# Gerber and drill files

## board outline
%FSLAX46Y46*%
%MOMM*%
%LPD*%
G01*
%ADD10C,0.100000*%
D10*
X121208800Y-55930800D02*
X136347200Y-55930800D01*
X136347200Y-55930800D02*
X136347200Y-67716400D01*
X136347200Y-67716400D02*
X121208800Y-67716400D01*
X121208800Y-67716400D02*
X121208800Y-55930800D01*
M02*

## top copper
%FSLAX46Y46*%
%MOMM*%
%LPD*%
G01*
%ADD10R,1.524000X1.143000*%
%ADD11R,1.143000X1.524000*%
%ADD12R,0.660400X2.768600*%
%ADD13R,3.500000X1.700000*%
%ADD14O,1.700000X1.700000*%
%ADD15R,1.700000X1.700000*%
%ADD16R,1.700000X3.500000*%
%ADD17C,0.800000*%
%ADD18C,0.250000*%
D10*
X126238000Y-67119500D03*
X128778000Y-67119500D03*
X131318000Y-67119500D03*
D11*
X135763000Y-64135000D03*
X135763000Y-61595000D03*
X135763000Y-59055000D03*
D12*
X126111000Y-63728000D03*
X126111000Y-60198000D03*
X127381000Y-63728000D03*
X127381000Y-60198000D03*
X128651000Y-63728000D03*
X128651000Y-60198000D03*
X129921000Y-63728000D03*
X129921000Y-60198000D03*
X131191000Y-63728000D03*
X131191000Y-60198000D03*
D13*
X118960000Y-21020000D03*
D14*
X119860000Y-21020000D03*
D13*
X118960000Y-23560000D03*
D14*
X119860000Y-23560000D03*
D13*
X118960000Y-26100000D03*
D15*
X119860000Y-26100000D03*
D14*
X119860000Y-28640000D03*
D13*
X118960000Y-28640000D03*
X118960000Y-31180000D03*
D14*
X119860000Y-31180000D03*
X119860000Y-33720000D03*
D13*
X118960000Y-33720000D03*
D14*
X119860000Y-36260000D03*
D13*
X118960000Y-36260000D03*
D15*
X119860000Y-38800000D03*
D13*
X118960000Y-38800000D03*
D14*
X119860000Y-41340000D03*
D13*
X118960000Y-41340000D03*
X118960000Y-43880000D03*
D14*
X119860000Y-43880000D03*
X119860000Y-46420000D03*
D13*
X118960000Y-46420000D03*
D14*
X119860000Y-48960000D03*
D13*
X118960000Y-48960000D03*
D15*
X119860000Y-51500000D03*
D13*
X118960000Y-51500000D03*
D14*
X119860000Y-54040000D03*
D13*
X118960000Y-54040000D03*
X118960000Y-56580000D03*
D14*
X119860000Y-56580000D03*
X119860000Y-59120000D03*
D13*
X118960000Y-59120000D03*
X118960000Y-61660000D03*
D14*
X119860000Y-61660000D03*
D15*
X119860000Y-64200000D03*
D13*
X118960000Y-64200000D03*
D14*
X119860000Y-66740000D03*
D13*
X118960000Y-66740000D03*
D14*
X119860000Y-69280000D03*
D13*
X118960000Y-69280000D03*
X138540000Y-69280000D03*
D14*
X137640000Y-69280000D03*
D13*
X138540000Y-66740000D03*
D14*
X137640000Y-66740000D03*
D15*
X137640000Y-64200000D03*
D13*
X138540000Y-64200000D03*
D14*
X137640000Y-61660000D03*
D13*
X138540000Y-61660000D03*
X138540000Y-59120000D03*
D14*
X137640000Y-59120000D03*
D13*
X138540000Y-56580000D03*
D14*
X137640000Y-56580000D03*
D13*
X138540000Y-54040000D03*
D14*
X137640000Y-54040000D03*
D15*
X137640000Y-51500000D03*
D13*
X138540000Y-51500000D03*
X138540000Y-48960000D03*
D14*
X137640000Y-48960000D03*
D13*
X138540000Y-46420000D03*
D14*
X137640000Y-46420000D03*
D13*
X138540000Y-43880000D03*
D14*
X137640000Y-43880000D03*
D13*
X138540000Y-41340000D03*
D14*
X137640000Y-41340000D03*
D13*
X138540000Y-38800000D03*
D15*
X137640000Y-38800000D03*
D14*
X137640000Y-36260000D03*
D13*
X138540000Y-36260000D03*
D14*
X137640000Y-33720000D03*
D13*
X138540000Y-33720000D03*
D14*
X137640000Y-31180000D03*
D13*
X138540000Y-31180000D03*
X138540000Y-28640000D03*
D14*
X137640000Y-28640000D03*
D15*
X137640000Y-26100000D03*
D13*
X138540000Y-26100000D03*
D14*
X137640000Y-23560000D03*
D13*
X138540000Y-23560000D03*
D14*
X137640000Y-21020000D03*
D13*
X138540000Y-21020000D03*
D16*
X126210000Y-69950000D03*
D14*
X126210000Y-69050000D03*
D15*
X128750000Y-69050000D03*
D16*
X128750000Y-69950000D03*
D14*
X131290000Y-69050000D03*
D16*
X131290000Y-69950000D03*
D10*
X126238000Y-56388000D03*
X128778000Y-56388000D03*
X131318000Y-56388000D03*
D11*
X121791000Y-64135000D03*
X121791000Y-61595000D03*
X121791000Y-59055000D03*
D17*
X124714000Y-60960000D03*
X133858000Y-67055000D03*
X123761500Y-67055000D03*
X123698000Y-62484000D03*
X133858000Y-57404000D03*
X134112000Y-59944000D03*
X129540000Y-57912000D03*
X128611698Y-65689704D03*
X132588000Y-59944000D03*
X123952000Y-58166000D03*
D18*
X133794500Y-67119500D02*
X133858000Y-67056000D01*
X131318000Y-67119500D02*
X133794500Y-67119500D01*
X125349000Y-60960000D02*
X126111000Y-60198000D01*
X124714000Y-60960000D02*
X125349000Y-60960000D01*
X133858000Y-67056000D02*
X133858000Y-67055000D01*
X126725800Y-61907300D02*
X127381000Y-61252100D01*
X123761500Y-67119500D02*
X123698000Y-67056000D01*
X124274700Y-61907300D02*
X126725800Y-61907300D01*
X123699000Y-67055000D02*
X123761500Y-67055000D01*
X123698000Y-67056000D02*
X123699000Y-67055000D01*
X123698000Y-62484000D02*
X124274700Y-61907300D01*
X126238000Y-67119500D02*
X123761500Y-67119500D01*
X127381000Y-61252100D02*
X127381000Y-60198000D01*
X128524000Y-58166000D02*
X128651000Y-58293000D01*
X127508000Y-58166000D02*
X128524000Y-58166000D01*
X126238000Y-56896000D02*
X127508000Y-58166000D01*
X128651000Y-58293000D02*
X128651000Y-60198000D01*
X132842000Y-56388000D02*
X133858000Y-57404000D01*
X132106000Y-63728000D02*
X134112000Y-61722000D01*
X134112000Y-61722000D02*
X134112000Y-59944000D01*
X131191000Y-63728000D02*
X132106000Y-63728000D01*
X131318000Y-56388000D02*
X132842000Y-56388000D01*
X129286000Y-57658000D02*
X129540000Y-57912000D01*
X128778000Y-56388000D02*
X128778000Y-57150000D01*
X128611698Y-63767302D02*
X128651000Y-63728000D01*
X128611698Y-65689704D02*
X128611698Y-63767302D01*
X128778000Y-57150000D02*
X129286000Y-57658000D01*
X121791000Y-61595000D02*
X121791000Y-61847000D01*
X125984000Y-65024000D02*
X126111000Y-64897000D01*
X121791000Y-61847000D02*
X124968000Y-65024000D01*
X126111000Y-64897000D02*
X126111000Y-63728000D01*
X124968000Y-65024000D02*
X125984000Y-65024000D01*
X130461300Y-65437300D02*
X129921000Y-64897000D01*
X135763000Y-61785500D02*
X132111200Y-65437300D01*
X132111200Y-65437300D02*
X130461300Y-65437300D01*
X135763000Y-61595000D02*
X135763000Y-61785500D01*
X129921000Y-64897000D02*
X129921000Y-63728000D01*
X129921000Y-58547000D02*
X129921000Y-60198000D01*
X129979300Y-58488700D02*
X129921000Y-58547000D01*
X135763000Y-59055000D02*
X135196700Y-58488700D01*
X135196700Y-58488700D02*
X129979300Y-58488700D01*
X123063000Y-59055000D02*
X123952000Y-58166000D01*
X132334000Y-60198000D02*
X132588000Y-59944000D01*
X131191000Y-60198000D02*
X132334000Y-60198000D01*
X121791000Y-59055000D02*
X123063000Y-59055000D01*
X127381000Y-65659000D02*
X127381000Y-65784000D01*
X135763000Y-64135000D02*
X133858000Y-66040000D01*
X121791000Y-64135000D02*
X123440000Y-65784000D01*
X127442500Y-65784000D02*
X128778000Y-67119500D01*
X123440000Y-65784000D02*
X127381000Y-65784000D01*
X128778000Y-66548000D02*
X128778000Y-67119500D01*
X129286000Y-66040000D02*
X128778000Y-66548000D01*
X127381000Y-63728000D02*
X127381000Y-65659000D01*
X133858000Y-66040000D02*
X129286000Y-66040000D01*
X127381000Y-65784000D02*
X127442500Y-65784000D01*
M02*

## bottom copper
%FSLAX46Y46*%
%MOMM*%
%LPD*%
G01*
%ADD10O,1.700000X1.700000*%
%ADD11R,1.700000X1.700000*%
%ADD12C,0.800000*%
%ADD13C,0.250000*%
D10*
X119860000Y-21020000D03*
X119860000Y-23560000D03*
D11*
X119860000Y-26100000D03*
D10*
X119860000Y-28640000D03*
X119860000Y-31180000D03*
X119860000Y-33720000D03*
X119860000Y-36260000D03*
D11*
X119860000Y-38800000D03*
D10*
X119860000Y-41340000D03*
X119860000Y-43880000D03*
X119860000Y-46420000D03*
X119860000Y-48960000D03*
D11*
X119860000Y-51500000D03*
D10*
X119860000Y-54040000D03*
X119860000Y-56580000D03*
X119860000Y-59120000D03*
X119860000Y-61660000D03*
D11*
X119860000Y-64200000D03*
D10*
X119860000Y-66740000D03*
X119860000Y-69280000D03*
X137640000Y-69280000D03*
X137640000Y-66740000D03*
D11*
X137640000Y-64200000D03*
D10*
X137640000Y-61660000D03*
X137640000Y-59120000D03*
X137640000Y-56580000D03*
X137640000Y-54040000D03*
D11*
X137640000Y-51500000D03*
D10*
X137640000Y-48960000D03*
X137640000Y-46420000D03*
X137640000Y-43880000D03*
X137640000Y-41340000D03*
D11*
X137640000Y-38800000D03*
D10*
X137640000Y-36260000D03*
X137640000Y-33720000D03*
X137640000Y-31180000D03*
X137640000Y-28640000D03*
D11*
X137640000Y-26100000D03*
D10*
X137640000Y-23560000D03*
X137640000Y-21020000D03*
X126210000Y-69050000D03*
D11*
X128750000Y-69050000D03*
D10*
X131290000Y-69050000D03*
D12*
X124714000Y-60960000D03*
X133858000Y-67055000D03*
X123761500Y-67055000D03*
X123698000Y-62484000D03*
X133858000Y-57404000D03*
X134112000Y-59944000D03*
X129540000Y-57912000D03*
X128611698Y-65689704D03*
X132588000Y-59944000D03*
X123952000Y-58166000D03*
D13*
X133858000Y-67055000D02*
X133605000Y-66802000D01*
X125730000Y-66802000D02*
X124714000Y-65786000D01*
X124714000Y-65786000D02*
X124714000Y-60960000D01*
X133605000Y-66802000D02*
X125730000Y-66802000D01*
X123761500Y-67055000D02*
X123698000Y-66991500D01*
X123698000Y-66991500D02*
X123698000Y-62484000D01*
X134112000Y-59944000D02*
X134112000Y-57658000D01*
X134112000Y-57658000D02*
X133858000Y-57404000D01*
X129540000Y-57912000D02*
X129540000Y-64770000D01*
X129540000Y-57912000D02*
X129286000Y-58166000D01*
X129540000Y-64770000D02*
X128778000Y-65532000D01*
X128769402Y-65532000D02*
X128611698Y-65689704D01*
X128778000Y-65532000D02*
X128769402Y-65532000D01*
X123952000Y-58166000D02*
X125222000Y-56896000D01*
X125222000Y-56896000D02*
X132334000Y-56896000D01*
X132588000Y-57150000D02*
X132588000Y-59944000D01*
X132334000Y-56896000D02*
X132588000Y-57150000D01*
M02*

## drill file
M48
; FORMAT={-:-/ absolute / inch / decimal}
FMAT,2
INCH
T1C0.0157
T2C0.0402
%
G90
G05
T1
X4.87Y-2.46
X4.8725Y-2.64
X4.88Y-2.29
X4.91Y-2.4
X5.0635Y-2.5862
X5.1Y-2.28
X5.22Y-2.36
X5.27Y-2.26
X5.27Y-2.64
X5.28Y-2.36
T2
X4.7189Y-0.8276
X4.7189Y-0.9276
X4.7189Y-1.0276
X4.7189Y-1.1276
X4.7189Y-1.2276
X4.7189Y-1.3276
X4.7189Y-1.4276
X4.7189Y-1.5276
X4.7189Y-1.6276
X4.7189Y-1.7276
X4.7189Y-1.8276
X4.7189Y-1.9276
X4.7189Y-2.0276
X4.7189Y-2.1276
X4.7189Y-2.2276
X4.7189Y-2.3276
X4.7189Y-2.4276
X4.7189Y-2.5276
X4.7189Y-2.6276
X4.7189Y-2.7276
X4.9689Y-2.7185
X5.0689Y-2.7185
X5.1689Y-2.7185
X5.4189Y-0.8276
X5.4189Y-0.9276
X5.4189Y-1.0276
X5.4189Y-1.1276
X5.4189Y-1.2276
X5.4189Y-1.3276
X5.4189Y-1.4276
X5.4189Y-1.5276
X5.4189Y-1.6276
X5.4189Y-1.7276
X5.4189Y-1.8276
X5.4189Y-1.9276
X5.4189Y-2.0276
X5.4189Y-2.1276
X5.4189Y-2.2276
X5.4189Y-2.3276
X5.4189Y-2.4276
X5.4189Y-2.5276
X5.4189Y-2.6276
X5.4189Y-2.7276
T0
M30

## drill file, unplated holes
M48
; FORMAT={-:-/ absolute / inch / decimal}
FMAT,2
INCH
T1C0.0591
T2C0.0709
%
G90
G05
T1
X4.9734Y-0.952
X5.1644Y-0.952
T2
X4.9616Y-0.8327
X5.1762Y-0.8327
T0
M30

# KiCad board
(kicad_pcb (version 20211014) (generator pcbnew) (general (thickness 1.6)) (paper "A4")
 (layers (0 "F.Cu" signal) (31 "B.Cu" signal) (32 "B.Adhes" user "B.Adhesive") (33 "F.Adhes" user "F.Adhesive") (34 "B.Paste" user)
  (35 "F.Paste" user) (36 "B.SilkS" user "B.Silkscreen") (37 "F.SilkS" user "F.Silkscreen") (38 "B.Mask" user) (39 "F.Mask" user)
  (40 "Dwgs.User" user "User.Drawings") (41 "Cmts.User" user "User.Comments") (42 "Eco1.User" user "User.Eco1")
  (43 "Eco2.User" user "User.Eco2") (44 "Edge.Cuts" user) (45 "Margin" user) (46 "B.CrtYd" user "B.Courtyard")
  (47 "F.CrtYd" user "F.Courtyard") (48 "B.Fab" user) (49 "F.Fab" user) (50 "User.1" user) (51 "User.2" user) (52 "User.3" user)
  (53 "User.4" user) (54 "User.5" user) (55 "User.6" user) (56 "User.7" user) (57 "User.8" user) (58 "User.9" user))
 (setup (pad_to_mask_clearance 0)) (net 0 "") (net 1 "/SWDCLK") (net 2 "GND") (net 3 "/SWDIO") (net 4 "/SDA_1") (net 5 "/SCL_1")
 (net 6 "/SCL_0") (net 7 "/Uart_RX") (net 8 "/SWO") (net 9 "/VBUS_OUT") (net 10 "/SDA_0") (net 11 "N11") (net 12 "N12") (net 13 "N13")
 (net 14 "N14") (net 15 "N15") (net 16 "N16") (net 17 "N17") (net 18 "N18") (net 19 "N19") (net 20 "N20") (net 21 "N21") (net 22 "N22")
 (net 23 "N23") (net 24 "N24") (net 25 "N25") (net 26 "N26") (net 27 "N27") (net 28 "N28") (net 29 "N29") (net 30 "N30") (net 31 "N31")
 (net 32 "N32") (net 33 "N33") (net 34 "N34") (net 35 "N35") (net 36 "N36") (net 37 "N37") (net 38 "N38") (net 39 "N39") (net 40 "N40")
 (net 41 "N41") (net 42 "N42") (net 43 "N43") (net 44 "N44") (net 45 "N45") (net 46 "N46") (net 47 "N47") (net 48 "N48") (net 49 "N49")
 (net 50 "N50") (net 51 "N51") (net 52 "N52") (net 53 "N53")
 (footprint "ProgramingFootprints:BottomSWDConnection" (layer "F.Cu") (at 128.778 66.548)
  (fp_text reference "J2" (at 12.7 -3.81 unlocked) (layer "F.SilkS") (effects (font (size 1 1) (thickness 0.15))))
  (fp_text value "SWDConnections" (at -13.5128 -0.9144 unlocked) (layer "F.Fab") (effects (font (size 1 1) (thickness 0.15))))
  (pad "1" smd rect (at -2.54 0.5715 90) (size 1.143 1.524) (layers "F.Cu" "F.Paste" "F.Mask") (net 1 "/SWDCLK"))
  (pad "2" smd rect (at 0 0.5715 90) (size 1.143 1.524) (layers "F.Cu" "F.Paste" "F.Mask") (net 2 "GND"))
  (pad "3" smd rect (at 2.54 0.5715 90) (size 1.143 1.524) (layers "F.Cu" "F.Paste" "F.Mask") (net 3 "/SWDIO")))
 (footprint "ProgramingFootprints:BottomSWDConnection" (layer "F.Cu") (at 135.1915 61.595 90)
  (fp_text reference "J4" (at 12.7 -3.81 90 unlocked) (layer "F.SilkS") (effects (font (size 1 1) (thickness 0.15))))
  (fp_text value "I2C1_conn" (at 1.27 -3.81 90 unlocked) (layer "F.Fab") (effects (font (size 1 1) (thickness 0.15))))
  (pad "1" smd rect (at -2.54 0.5715 180) (size 1.143 1.524) (layers "F.Cu" "F.Paste" "F.Mask") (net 2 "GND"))
  (pad "2" smd rect (at 0 0.5715 180) (size 1.143 1.524) (layers "F.Cu" "F.Paste" "F.Mask") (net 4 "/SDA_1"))
  (pad "3" smd rect (at 2.54 0.5715 180) (size 1.143 1.524) (layers "F.Cu" "F.Paste" "F.Mask") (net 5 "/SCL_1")))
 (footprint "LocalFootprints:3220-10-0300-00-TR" (layer "F.Cu") (at 128.651 61.963)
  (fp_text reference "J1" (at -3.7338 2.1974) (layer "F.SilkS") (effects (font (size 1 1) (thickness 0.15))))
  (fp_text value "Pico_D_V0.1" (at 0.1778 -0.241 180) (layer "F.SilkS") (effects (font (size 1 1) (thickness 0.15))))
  (pad "1" smd rect (at -2.54 1.765) (size 0.6604 2.7686) (layers "F.Cu" "F.Paste" "F.Mask") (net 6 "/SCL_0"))
  (pad "2" smd rect (at -2.54 -1.765) (size 0.6604 2.7686) (layers "F.Cu" "F.Paste" "F.Mask") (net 3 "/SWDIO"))
  (pad "3" smd rect (at -1.27 1.765) (size 0.6604 2.7686) (layers "F.Cu" "F.Paste" "F.Mask") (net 2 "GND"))
  (pad "4" smd rect (at -1.27 -1.765) (size 0.6604 2.7686) (layers "F.Cu" "F.Paste" "F.Mask") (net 1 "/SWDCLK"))
  (pad "5" smd rect (at 0 1.765) (size 0.6604 2.7686) (layers "F.Cu" "F.Paste" "F.Mask") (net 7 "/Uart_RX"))
  (pad "6" smd rect (at 0 -1.765) (size 0.6604 2.7686) (layers "F.Cu" "F.Paste" "F.Mask") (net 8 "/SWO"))
  (pad "7" smd rect (at 1.27 1.765) (size 0.6604 2.7686) (layers "F.Cu" "F.Paste" "F.Mask") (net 4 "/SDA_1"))
  (pad "8" smd rect (at 1.27 -1.765) (size 0.6604 2.7686) (layers "F.Cu" "F.Paste" "F.Mask") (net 5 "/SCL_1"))
  (pad "9" smd rect (at 2.54 1.765) (size 0.6604 2.7686) (layers "F.Cu" "F.Paste" "F.Mask") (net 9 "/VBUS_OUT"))
  (pad "10" smd rect (at 2.54 -1.765) (size 0.6604 2.7686) (layers "F.Cu" "F.Paste" "F.Mask") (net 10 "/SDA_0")))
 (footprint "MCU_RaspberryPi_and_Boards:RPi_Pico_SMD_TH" (layer "F.Cu") (at 128.75 45.15)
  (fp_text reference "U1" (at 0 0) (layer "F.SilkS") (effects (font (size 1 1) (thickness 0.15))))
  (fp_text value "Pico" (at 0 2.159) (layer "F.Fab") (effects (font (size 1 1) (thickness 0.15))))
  (pad "" np_thru_hole oval (at 2.425 -20.97) (size 1.5 1.5) (drill 1.5) (layers *.Cu *.Mask))
  (pad "" np_thru_hole oval (at -2.425 -20.97) (size 1.5 1.5) (drill 1.5) (layers *.Cu *.Mask))
  (pad "" np_thru_hole oval (at -2.725 -24) (size 1.8 1.8) (drill 1.8) (layers *.Cu *.Mask))
  (pad "" np_thru_hole oval (at 2.725 -24) (size 1.8 1.8) (drill 1.8) (layers *.Cu *.Mask))
  (pad "1" smd rect (at -8.89 -24.13) (size 3.5 1.7) (drill (offset -0.9 0)) (layers "F.Cu" "F.Mask") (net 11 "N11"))
  (pad "1" thru_hole oval (at -8.89 -24.13) (size 1.7 1.7) (drill 1.02) (layers *.Cu *.Mask) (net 11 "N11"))
  (pad "2" smd rect (at -8.89 -21.59) (size 3.5 1.7) (drill (offset -0.9 0)) (layers "F.Cu" "F.Mask") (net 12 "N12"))
  (pad "2" thru_hole oval (at -8.89 -21.59) (size 1.7 1.7) (drill 1.02) (layers *.Cu *.Mask) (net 12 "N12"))
  (pad "3" smd rect (at -8.89 -19.05) (size 3.5 1.7) (drill (offset -0.9 0)) (layers "F.Cu" "F.Mask") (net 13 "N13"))
  (pad "3" thru_hole rect (at -8.89 -19.05) (size 1.7 1.7) (drill 1.02) (layers *.Cu *.Mask) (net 13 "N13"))
  (pad "4" thru_hole oval (at -8.89 -16.51) (size 1.7 1.7) (drill 1.02) (layers *.Cu *.Mask) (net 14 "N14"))
  (pad "4" smd rect (at -8.89 -16.51) (size 3.5 1.7) (drill (offset -0.9 0)) (layers "F.Cu" "F.Mask") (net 14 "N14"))
  (pad "5" smd rect (at -8.89 -13.97) (size 3.5 1.7) (drill (offset -0.9 0)) (layers "F.Cu" "F.Mask") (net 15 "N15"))
  (pad "5" thru_hole oval (at -8.89 -13.97) (size 1.7 1.7) (drill 1.02) (layers *.Cu *.Mask) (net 15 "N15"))
  (pad "6" thru_hole oval (at -8.89 -11.43) (size 1.7 1.7) (drill 1.02) (layers *.Cu *.Mask) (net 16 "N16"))
  (pad "6" smd rect (at -8.89 -11.43) (size 3.5 1.7) (drill (offset -0.9 0)) (layers "F.Cu" "F.Mask") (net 16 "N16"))
  (pad "7" thru_hole oval (at -8.89 -8.89) (size 1.7 1.7) (drill 1.02) (layers *.Cu *.Mask) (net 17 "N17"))
  (pad "7" smd rect (at -8.89 -8.89) (size 3.5 1.7) (drill (offset -0.9 0)) (layers "F.Cu" "F.Mask") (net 17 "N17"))
  (pad "8" thru_hole rect (at -8.89 -6.35) (size 1.7 1.7) (drill 1.02) (layers *.Cu *.Mask) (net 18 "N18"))
  (pad "8" smd rect (at -8.89 -6.35) (size 3.5 1.7) (drill (offset -0.9 0)) (layers "F.Cu" "F.Mask") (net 18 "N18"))
  (pad "9" thru_hole oval (at -8.89 -3.81) (size 1.7 1.7) (drill 1.02) (layers *.Cu *.Mask) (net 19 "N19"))
  (pad "9" smd rect (at -8.89 -3.81) (size 3.5 1.7) (drill (offset -0.9 0)) (layers "F.Cu" "F.Mask") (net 19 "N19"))
  (pad "10" smd rect (at -8.89 -1.27) (size 3.5 1.7) (drill (offset -0.9 0)) (layers "F.Cu" "F.Mask") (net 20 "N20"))
  (pad "10" thru_hole oval (at -8.89 -1.27) (size 1.7 1.7) (drill 1.02) (layers *.Cu *.Mask) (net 20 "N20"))
  (pad "11" thru_hole oval (at -8.89 1.27) (size 1.7 1.7) (drill 1.02) (layers *.Cu *.Mask) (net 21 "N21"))
  (pad "11" smd rect (at -8.89 1.27) (size 3.5 1.7) (drill (offset -0.9 0)) (layers "F.Cu" "F.Mask") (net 21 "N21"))
  (pad "12" thru_hole oval (at -8.89 3.81) (size 1.7 1.7) (drill 1.02) (layers *.Cu *.Mask) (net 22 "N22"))
  (pad "12" smd rect (at -8.89 3.81) (size 3.5 1.7) (drill (offset -0.9 0)) (layers "F.Cu" "F.Mask") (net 22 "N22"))
  (pad "13" thru_hole rect (at -8.89 6.35) (size 1.7 1.7) (drill 1.02) (layers *.Cu *.Mask) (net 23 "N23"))
  (pad "13" smd rect (at -8.89 6.35) (size 3.5 1.7) (drill (offset -0.9 0)) (layers "F.Cu" "F.Mask") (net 23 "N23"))
  (pad "14" thru_hole oval (at -8.89 8.89) (size 1.7 1.7) (drill 1.02) (layers *.Cu *.Mask) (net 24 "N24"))
  (pad "14" smd rect (at -8.89 8.89) (size 3.5 1.7) (drill (offset -0.9 0)) (layers "F.Cu" "F.Mask") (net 24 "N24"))
  (pad "15" smd rect (at -8.89 11.43) (size 3.5 1.7) (drill (offset -0.9 0)) (layers "F.Cu" "F.Mask") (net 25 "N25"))
  (pad "15" thru_hole oval (at -8.89 11.43) (size 1.7 1.7) (drill 1.02) (layers *.Cu *.Mask) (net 25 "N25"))
  (pad "16" thru_hole oval (at -8.89 13.97) (size 1.7 1.7) (drill 1.02) (layers *.Cu *.Mask) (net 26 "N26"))
  (pad "16" smd rect (at -8.89 13.97) (size 3.5 1.7) (drill (offset -0.9 0)) (layers "F.Cu" "F.Mask") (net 26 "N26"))
  (pad "17" smd rect (at -8.89 16.51) (size 3.5 1.7) (drill (offset -0.9 0)) (layers "F.Cu" "F.Mask") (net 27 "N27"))
  (pad "17" thru_hole oval (at -8.89 16.51) (size 1.7 1.7) (drill 1.02) (layers *.Cu *.Mask) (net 27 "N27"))
  (pad "18" thru_hole rect (at -8.89 19.05) (size 1.7 1.7) (drill 1.02) (layers *.Cu *.Mask) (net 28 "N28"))
  (pad "18" smd rect (at -8.89 19.05) (size 3.5 1.7) (drill (offset -0.9 0)) (layers "F.Cu" "F.Mask") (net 28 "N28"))
  (pad "19" thru_hole oval (at -8.89 21.59) (size 1.7 1.7) (drill 1.02) (layers *.Cu *.Mask) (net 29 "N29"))
  (pad "19" smd rect (at -8.89 21.59) (size 3.5 1.7) (drill (offset -0.9 0)) (layers "F.Cu" "F.Mask") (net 29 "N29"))
  (pad "20" thru_hole oval (at -8.89 24.13) (size 1.7 1.7) (drill 1.02) (layers *.Cu *.Mask) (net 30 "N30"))
  (pad "20" smd rect (at -8.89 24.13) (size 3.5 1.7) (drill (offset -0.9 0)) (layers "F.Cu" "F.Mask") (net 30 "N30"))
  (pad "21" smd rect (at 8.89 24.13) (size 3.5 1.7) (drill (offset 0.9 0)) (layers "F.Cu" "F.Mask") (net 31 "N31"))
  (pad "21" thru_hole oval (at 8.89 24.13) (size 1.7 1.7) (drill 1.02) (layers *.Cu *.Mask) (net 31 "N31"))
  (pad "22" smd rect (at 8.89 21.59) (size 3.5 1.7) (drill (offset 0.9 0)) (layers "F.Cu" "F.Mask") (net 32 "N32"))
  (pad "22" thru_hole oval (at 8.89 21.59) (size 1.7 1.7) (drill 1.02) (layers *.Cu *.Mask) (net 32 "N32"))
  (pad "23" thru_hole rect (at 8.89 19.05) (size 1.7 1.7) (drill 1.02) (layers *.Cu *.Mask) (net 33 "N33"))
  (pad "23" smd rect (at 8.89 19.05) (size 3.5 1.7) (drill (offset 0.9 0)) (layers "F.Cu" "F.Mask") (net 33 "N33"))
  (pad "24" thru_hole oval (at 8.89 16.51) (size 1.7 1.7) (drill 1.02) (layers *.Cu *.Mask) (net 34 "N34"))
  (pad "24" smd rect (at 8.89 16.51) (size 3.5 1.7) (drill (offset 0.9 0)) (layers "F.Cu" "F.Mask") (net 34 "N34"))
  (pad "25" smd rect (at 8.89 13.97) (size 3.5 1.7) (drill (offset 0.9 0)) (layers "F.Cu" "F.Mask") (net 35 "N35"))
  (pad "25" thru_hole oval (at 8.89 13.97) (size 1.7 1.7) (drill 1.02) (layers *.Cu *.Mask) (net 35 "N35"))
  (pad "26" smd rect (at 8.89 11.43) (size 3.5 1.7) (drill (offset 0.9 0)) (layers "F.Cu" "F.Mask") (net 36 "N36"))
  (pad "26" thru_hole oval (at 8.89 11.43) (size 1.7 1.7) (drill 1.02) (layers *.Cu *.Mask) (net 36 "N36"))
  (pad "27" smd rect (at 8.89 8.89) (size 3.5 1.7) (drill (offset 0.9 0)) (layers "F.Cu" "F.Mask") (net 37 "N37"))
  (pad "27" thru_hole oval (at 8.89 8.89) (size 1.7 1.7) (drill 1.02) (layers *.Cu *.Mask) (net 37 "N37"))
  (pad "28" thru_hole rect (at 8.89 6.35) (size 1.7 1.7) (drill 1.02) (layers *.Cu *.Mask) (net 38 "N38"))
  (pad "28" smd rect (at 8.89 6.35) (size 3.5 1.7) (drill (offset 0.9 0)) (layers "F.Cu" "F.Mask") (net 38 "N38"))
  (pad "29" smd rect (at 8.89 3.81) (size 3.5 1.7) (drill (offset 0.9 0)) (layers "F.Cu" "F.Mask") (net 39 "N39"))
  (pad "29" thru_hole oval (at 8.89 3.81) (size 1.7 1.7) (drill 1.02) (layers *.Cu *.Mask) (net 39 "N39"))
  (pad "30" smd rect (at 8.89 1.27) (size 3.5 1.7) (drill (offset 0.9 0)) (layers "F.Cu" "F.Mask") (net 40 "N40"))
  (pad "30" thru_hole oval (at 8.89 1.27) (size 1.7 1.7) (drill 1.02) (layers *.Cu *.Mask) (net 40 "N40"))
  (pad "31" smd rect (at 8.89 -1.27) (size 3.5 1.7) (drill (offset 0.9 0)) (layers "F.Cu" "F.Mask") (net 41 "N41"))
  (pad "31" thru_hole oval (at 8.89 -1.27) (size 1.7 1.7) (drill 1.02) (layers *.Cu *.Mask) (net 41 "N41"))
  (pad "32" smd rect (at 8.89 -3.81) (size 3.5 1.7) (drill (offset 0.9 0)) (layers "F.Cu" "F.Mask") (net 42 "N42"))
  (pad "32" thru_hole oval (at 8.89 -3.81) (size 1.7 1.7) (drill 1.02) (layers *.Cu *.Mask) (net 42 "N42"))
  (pad "33" smd rect (at 8.89 -6.35) (size 3.5 1.7) (drill (offset 0.9 0)) (layers "F.Cu" "F.Mask") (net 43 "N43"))
  (pad "33" thru_hole rect (at 8.89 -6.35) (size 1.7 1.7) (drill 1.02) (layers *.Cu *.Mask) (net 43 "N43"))
  (pad "34" thru_hole oval (at 8.89 -8.89) (size 1.7 1.7) (drill 1.02) (layers *.Cu *.Mask) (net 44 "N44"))
  (pad "34" smd rect (at 8.89 -8.89) (size 3.5 1.7) (drill (offset 0.9 0)) (layers "F.Cu" "F.Mask") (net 44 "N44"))
  (pad "35" thru_hole oval (at 8.89 -11.43) (size 1.7 1.7) (drill 1.02) (layers *.Cu *.Mask) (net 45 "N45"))
  (pad "35" smd rect (at 8.89 -11.43) (size 3.5 1.7) (drill (offset 0.9 0)) (layers "F.Cu" "F.Mask") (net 45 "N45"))
  (pad "36" thru_hole oval (at 8.89 -13.97) (size 1.7 1.7) (drill 1.02) (layers *.Cu *.Mask) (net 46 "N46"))
  (pad "36" smd rect (at 8.89 -13.97) (size 3.5 1.7) (drill (offset 0.9 0)) (layers "F.Cu" "F.Mask") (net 46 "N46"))
  (pad "37" smd rect (at 8.89 -16.51) (size 3.5 1.7) (drill (offset 0.9 0)) (layers "F.Cu" "F.Mask") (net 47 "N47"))
  (pad "37" thru_hole oval (at 8.89 -16.51) (size 1.7 1.7) (drill 1.02) (layers *.Cu *.Mask) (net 47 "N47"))
  (pad "38" thru_hole rect (at 8.89 -19.05) (size 1.7 1.7) (drill 1.02) (layers *.Cu *.Mask) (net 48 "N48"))
  (pad "38" smd rect (at 8.89 -19.05) (size 3.5 1.7) (drill (offset 0.9 0)) (layers "F.Cu" "F.Mask") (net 48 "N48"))
  (pad "39" thru_hole oval (at 8.89 -21.59) (size 1.7 1.7) (drill 1.02) (layers *.Cu *.Mask) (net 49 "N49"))
  (pad "39" smd rect (at 8.89 -21.59) (size 3.5 1.7) (drill (offset 0.9 0)) (layers "F.Cu" "F.Mask") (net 49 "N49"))
  (pad "40" thru_hole oval (at 8.89 -24.13) (size 1.7 1.7) (drill 1.02) (layers *.Cu *.Mask) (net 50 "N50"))
  (pad "40" smd rect (at 8.89 -24.13) (size 3.5 1.7) (drill (offset 0.9 0)) (layers "F.Cu" "F.Mask") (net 50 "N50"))
  (pad "41" smd rect (at -2.54 23.9 90) (size 3.5 1.7) (drill (offset -0.9 0)) (layers "F.Cu" "F.Mask") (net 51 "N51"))
  (pad "41" thru_hole oval (at -2.54 23.9) (size 1.7 1.7) (drill 1.02) (layers *.Cu *.Mask) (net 51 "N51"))
  (pad "42" thru_hole rect (at 0 23.9) (size 1.7 1.7) (drill 1.02) (layers *.Cu *.Mask) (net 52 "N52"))
  (pad "42" smd rect (at 0 23.9 90) (size 3.5 1.7) (drill (offset -0.9 0)) (layers "F.Cu" "F.Mask") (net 52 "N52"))
  (pad "43" thru_hole oval (at 2.54 23.9) (size 1.7 1.7) (drill 1.02) (layers *.Cu *.Mask) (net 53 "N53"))
  (pad "43" smd rect (at 2.54 23.9 90) (size 3.5 1.7) (drill (offset -0.9 0)) (layers "F.Cu" "F.Mask") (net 53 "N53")))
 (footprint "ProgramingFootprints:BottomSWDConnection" (layer "F.Cu") (at 128.778 55.8165)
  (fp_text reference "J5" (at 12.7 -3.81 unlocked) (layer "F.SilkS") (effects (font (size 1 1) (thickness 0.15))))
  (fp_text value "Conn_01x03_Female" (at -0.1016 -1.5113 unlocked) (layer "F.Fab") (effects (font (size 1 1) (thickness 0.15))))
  (pad "1" smd rect (at -2.54 0.5715 90) (size 1.143 1.524) (layers "F.Cu" "F.Paste" "F.Mask") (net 8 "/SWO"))
  (pad "2" smd rect (at 0 0.5715 90) (size 1.143 1.524) (layers "F.Cu" "F.Paste" "F.Mask") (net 7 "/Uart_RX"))
  (pad "3" smd rect (at 2.54 0.5715 90) (size 1.143 1.524) (layers "F.Cu" "F.Paste" "F.Mask") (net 9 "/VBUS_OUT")))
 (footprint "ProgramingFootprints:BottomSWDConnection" (layer "F.Cu") (at 121.2195 61.595 90)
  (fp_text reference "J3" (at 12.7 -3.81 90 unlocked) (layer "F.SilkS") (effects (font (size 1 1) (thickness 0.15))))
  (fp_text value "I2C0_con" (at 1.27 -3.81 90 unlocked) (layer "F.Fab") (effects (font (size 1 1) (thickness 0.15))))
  (pad "1" smd rect (at -2.54 0.5715 180) (size 1.143 1.524) (layers "F.Cu" "F.Paste" "F.Mask") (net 2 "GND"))
  (pad "2" smd rect (at 0 0.5715 180) (size 1.143 1.524) (layers "F.Cu" "F.Paste" "F.Mask") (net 6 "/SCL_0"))
  (pad "3" smd rect (at 2.54 0.5715 180) (size 1.143 1.524) (layers "F.Cu" "F.Paste" "F.Mask") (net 10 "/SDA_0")))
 (gr_rect (start 121.2088 55.9308) (end 136.3472 67.7164) (layer "Edge.Cuts") (width 0.1) (fill none))
 (segment (start 133.7945 67.1195) (end 133.858 67.056) (width 0.25) (layer "F.Cu") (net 3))
 (segment (start 131.318 67.1195) (end 133.7945 67.1195) (width 0.25) (layer "F.Cu") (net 3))
 (segment (start 125.349 60.96) (end 126.111 60.198) (width 0.25) (layer "F.Cu") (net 3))
 (segment (start 124.714 60.96) (end 125.349 60.96) (width 0.25) (layer "F.Cu") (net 3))
 (segment (start 133.858 67.056) (end 133.858 67.055) (width 0.25) (layer "F.Cu") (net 3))
 (via (at 124.714 60.96) (size 0.8) (drill 0.4) (layers "F.Cu" "B.Cu") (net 3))
 (via (at 133.858 67.055) (size 0.8) (drill 0.4) (layers "F.Cu" "B.Cu") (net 3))
 (segment (start 133.858 67.055) (end 133.605 66.802) (width 0.25) (layer "B.Cu") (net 3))
 (segment (start 125.73 66.802) (end 124.714 65.786) (width 0.25) (layer "B.Cu") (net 3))
 (segment (start 124.714 65.786) (end 124.714 60.96) (width 0.25) (layer "B.Cu") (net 3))
 (segment (start 133.605 66.802) (end 125.73 66.802) (width 0.25) (layer "B.Cu") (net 3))
 (segment (start 126.7258 61.9073) (end 127.381 61.2521) (width 0.25) (layer "F.Cu") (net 1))
 (segment (start 123.7615 67.1195) (end 123.698 67.056) (width 0.25) (layer "F.Cu") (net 1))
 (segment (start 124.2747 61.9073) (end 126.7258 61.9073) (width 0.25) (layer "F.Cu") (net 1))
 (segment (start 123.699 67.055) (end 123.7615 67.055) (width 0.25) (layer "F.Cu") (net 1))
 (segment (start 123.698 67.056) (end 123.699 67.055) (width 0.25) (layer "F.Cu") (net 1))
 (segment (start 123.698 62.484) (end 124.2747 61.9073) (width 0.25) (layer "F.Cu") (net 1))
 (segment (start 126.238 67.1195) (end 123.7615 67.1195) (width 0.25) (layer "F.Cu") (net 1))
 (segment (start 127.381 61.2521) (end 127.381 60.198) (width 0.25) (layer "F.Cu") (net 1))
 (via (at 123.7615 67.055) (size 0.8) (drill 0.4) (layers "F.Cu" "B.Cu") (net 1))
 (via (at 123.698 62.484) (size 0.8) (drill 0.4) (layers "F.Cu" "B.Cu") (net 1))
 (segment (start 123.7615 67.055) (end 123.698 66.9915) (width 0.25) (layer "B.Cu") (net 1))
 (segment (start 123.698 66.9915) (end 123.698 62.484) (width 0.25) (layer "B.Cu") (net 1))
 (segment (start 128.524 58.166) (end 128.651 58.293) (width 0.25) (layer "F.Cu") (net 8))
 (segment (start 127.508 58.166) (end 128.524 58.166) (width 0.25) (layer "F.Cu") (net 8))
 (segment (start 126.238 56.896) (end 127.508 58.166) (width 0.25) (layer "F.Cu") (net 8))
 (segment (start 128.651 58.293) (end 128.651 60.198) (width 0.25) (layer "F.Cu") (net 8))
 (segment (start 132.842 56.388) (end 133.858 57.404) (width 0.25) (layer "F.Cu") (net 9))
 (segment (start 132.106 63.728) (end 134.112 61.722) (width 0.25) (layer "F.Cu") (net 9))
 (segment (start 134.112 61.722) (end 134.112 59.944) (width 0.25) (layer "F.Cu") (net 9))
 (segment (start 131.191 63.728) (end 132.106 63.728) (width 0.25) (layer "F.Cu") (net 9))
 (segment (start 131.318 56.388) (end 132.842 56.388) (width 0.25) (layer "F.Cu") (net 9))
 (via (at 133.858 57.404) (size 0.8) (drill 0.4) (layers "F.Cu" "B.Cu") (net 9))
 (via (at 134.112 59.944) (size 0.8) (drill 0.4) (layers "F.Cu" "B.Cu") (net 9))
 (segment (start 134.112 59.944) (end 134.112 57.658) (width 0.25) (layer "B.Cu") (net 9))
 (segment (start 134.112 57.658) (end 133.858 57.404) (width 0.25) (layer "B.Cu") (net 9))
 (segment (start 129.286 57.658) (end 129.54 57.912) (width 0.25) (layer "F.Cu") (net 7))
 (segment (start 128.778 56.388) (end 128.778 57.15) (width 0.25) (layer "F.Cu") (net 7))
 (segment (start 128.611698 63.767302) (end 128.651 63.728) (width 0.25) (layer "F.Cu") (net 7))
 (segment (start 128.611698 65.689704) (end 128.611698 63.767302) (width 0.25) (layer "F.Cu") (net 7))
 (segment (start 128.778 57.15) (end 129.286 57.658) (width 0.25) (layer "F.Cu") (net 7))
 (via (at 129.54 57.912) (size 0.8) (drill 0.4) (layers "F.Cu" "B.Cu") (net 7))
 (via (at 128.611698 65.689704) (size 0.8) (drill 0.4) (layers "F.Cu" "B.Cu") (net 7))
 (segment (start 129.54 57.912) (end 129.54 64.77) (width 0.25) (layer "B.Cu") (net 7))
 (segment (start 129.54 57.912) (end 129.286 58.166) (width 0.25) (layer "B.Cu") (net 7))
 (segment (start 129.54 64.77) (end 128.778 65.532) (width 0.25) (layer "B.Cu") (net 7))
 (segment (start 128.769402 65.532) (end 128.611698 65.689704) (width 0.25) (layer "B.Cu") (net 7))
 (segment (start 128.778 65.532) (end 128.769402 65.532) (width 0.25) (layer "B.Cu") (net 7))
 (segment (start 121.791 61.595) (end 121.791 61.847) (width 0.25) (layer "F.Cu") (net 6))
 (segment (start 125.984 65.024) (end 126.111 64.897) (width 0.25) (layer "F.Cu") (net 6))
 (segment (start 121.791 61.847) (end 124.968 65.024) (width 0.25) (layer "F.Cu") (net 6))
 (segment (start 126.111 64.897) (end 126.111 63.728) (width 0.25) (layer "F.Cu") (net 6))
 (segment (start 124.968 65.024) (end 125.984 65.024) (width 0.25) (layer "F.Cu") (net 6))
 (segment (start 130.4613 65.4373) (end 129.921 64.897) (width 0.25) (layer "F.Cu") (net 4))
 (segment (start 135.763 61.7855) (end 132.1112 65.4373) (width 0.25) (layer "F.Cu") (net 4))
 (segment (start 132.1112 65.4373) (end 130.4613 65.4373) (width 0.25) (layer "F.Cu") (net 4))
 (segment (start 135.763 61.595) (end 135.763 61.7855) (width 0.25) (layer "F.Cu") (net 4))
 (segment (start 129.921 64.897) (end 129.921 63.728) (width 0.25) (layer "F.Cu") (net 4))
 (segment (start 129.921 58.547) (end 129.921 60.198) (width 0.25) (layer "F.Cu") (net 5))
 (segment (start 129.9793 58.4887) (end 129.921 58.547) (width 0.25) (layer "F.Cu") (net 5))
 (segment (start 135.763 59.055) (end 135.1967 58.4887) (width 0.25) (layer "F.Cu") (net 5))
 (segment (start 135.1967 58.4887) (end 129.9793 58.4887) (width 0.25) (layer "F.Cu") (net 5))
 (segment (start 123.063 59.055) (end 123.952 58.166) (width 0.25) (layer "F.Cu") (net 10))
 (segment (start 132.334 60.198) (end 132.588 59.944) (width 0.25) (layer "F.Cu") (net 10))
 (segment (start 131.191 60.198) (end 132.334 60.198) (width 0.25) (layer "F.Cu") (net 10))
 (segment (start 121.791 59.055) (end 123.063 59.055) (width 0.25) (layer "F.Cu") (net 10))
 (via (at 132.588 59.944) (size 0.8) (drill 0.4) (layers "F.Cu" "B.Cu") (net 10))
 (via (at 123.952 58.166) (size 0.8) (drill 0.4) (layers "F.Cu" "B.Cu") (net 10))
 (segment (start 123.952 58.166) (end 125.222 56.896) (width 0.25) (layer "B.Cu") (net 10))
 (segment (start 125.222 56.896) (end 132.334 56.896) (width 0.25) (layer "B.Cu") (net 10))
 (segment (start 132.588 57.15) (end 132.588 59.944) (width 0.25) (layer "B.Cu") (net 10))
 (segment (start 132.334 56.896) (end 132.588 57.15) (width 0.25) (layer "B.Cu") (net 10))
 (segment (start 127.381 65.659) (end 127.381 65.784) (width 0.25) (layer "F.Cu") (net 2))
 (segment (start 135.763 64.135) (end 133.858 66.04) (width 0.25) (layer "F.Cu") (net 2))
 (segment (start 121.791 64.135) (end 123.44 65.784) (width 0.25) (layer "F.Cu") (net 2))
 (segment (start 127.4425 65.784) (end 128.778 67.1195) (width 0.25) (layer "F.Cu") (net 2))
 (segment (start 123.44 65.784) (end 127.381 65.784) (width 0.25) (layer "F.Cu") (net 2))
 (segment (start 128.778 66.548) (end 128.778 67.1195) (width 0.25) (layer "F.Cu") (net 2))
 (segment (start 129.286 66.04) (end 128.778 66.548) (width 0.25) (layer "F.Cu") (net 2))
 (segment (start 127.381 63.728) (end 127.381 65.659) (width 0.25) (layer "F.Cu") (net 2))
 (segment (start 133.858 66.04) (end 129.286 66.04) (width 0.25) (layer "F.Cu") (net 2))
 (segment (start 127.381 65.784) (end 127.4425 65.784) (width 0.25) (layer "F.Cu") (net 2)))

